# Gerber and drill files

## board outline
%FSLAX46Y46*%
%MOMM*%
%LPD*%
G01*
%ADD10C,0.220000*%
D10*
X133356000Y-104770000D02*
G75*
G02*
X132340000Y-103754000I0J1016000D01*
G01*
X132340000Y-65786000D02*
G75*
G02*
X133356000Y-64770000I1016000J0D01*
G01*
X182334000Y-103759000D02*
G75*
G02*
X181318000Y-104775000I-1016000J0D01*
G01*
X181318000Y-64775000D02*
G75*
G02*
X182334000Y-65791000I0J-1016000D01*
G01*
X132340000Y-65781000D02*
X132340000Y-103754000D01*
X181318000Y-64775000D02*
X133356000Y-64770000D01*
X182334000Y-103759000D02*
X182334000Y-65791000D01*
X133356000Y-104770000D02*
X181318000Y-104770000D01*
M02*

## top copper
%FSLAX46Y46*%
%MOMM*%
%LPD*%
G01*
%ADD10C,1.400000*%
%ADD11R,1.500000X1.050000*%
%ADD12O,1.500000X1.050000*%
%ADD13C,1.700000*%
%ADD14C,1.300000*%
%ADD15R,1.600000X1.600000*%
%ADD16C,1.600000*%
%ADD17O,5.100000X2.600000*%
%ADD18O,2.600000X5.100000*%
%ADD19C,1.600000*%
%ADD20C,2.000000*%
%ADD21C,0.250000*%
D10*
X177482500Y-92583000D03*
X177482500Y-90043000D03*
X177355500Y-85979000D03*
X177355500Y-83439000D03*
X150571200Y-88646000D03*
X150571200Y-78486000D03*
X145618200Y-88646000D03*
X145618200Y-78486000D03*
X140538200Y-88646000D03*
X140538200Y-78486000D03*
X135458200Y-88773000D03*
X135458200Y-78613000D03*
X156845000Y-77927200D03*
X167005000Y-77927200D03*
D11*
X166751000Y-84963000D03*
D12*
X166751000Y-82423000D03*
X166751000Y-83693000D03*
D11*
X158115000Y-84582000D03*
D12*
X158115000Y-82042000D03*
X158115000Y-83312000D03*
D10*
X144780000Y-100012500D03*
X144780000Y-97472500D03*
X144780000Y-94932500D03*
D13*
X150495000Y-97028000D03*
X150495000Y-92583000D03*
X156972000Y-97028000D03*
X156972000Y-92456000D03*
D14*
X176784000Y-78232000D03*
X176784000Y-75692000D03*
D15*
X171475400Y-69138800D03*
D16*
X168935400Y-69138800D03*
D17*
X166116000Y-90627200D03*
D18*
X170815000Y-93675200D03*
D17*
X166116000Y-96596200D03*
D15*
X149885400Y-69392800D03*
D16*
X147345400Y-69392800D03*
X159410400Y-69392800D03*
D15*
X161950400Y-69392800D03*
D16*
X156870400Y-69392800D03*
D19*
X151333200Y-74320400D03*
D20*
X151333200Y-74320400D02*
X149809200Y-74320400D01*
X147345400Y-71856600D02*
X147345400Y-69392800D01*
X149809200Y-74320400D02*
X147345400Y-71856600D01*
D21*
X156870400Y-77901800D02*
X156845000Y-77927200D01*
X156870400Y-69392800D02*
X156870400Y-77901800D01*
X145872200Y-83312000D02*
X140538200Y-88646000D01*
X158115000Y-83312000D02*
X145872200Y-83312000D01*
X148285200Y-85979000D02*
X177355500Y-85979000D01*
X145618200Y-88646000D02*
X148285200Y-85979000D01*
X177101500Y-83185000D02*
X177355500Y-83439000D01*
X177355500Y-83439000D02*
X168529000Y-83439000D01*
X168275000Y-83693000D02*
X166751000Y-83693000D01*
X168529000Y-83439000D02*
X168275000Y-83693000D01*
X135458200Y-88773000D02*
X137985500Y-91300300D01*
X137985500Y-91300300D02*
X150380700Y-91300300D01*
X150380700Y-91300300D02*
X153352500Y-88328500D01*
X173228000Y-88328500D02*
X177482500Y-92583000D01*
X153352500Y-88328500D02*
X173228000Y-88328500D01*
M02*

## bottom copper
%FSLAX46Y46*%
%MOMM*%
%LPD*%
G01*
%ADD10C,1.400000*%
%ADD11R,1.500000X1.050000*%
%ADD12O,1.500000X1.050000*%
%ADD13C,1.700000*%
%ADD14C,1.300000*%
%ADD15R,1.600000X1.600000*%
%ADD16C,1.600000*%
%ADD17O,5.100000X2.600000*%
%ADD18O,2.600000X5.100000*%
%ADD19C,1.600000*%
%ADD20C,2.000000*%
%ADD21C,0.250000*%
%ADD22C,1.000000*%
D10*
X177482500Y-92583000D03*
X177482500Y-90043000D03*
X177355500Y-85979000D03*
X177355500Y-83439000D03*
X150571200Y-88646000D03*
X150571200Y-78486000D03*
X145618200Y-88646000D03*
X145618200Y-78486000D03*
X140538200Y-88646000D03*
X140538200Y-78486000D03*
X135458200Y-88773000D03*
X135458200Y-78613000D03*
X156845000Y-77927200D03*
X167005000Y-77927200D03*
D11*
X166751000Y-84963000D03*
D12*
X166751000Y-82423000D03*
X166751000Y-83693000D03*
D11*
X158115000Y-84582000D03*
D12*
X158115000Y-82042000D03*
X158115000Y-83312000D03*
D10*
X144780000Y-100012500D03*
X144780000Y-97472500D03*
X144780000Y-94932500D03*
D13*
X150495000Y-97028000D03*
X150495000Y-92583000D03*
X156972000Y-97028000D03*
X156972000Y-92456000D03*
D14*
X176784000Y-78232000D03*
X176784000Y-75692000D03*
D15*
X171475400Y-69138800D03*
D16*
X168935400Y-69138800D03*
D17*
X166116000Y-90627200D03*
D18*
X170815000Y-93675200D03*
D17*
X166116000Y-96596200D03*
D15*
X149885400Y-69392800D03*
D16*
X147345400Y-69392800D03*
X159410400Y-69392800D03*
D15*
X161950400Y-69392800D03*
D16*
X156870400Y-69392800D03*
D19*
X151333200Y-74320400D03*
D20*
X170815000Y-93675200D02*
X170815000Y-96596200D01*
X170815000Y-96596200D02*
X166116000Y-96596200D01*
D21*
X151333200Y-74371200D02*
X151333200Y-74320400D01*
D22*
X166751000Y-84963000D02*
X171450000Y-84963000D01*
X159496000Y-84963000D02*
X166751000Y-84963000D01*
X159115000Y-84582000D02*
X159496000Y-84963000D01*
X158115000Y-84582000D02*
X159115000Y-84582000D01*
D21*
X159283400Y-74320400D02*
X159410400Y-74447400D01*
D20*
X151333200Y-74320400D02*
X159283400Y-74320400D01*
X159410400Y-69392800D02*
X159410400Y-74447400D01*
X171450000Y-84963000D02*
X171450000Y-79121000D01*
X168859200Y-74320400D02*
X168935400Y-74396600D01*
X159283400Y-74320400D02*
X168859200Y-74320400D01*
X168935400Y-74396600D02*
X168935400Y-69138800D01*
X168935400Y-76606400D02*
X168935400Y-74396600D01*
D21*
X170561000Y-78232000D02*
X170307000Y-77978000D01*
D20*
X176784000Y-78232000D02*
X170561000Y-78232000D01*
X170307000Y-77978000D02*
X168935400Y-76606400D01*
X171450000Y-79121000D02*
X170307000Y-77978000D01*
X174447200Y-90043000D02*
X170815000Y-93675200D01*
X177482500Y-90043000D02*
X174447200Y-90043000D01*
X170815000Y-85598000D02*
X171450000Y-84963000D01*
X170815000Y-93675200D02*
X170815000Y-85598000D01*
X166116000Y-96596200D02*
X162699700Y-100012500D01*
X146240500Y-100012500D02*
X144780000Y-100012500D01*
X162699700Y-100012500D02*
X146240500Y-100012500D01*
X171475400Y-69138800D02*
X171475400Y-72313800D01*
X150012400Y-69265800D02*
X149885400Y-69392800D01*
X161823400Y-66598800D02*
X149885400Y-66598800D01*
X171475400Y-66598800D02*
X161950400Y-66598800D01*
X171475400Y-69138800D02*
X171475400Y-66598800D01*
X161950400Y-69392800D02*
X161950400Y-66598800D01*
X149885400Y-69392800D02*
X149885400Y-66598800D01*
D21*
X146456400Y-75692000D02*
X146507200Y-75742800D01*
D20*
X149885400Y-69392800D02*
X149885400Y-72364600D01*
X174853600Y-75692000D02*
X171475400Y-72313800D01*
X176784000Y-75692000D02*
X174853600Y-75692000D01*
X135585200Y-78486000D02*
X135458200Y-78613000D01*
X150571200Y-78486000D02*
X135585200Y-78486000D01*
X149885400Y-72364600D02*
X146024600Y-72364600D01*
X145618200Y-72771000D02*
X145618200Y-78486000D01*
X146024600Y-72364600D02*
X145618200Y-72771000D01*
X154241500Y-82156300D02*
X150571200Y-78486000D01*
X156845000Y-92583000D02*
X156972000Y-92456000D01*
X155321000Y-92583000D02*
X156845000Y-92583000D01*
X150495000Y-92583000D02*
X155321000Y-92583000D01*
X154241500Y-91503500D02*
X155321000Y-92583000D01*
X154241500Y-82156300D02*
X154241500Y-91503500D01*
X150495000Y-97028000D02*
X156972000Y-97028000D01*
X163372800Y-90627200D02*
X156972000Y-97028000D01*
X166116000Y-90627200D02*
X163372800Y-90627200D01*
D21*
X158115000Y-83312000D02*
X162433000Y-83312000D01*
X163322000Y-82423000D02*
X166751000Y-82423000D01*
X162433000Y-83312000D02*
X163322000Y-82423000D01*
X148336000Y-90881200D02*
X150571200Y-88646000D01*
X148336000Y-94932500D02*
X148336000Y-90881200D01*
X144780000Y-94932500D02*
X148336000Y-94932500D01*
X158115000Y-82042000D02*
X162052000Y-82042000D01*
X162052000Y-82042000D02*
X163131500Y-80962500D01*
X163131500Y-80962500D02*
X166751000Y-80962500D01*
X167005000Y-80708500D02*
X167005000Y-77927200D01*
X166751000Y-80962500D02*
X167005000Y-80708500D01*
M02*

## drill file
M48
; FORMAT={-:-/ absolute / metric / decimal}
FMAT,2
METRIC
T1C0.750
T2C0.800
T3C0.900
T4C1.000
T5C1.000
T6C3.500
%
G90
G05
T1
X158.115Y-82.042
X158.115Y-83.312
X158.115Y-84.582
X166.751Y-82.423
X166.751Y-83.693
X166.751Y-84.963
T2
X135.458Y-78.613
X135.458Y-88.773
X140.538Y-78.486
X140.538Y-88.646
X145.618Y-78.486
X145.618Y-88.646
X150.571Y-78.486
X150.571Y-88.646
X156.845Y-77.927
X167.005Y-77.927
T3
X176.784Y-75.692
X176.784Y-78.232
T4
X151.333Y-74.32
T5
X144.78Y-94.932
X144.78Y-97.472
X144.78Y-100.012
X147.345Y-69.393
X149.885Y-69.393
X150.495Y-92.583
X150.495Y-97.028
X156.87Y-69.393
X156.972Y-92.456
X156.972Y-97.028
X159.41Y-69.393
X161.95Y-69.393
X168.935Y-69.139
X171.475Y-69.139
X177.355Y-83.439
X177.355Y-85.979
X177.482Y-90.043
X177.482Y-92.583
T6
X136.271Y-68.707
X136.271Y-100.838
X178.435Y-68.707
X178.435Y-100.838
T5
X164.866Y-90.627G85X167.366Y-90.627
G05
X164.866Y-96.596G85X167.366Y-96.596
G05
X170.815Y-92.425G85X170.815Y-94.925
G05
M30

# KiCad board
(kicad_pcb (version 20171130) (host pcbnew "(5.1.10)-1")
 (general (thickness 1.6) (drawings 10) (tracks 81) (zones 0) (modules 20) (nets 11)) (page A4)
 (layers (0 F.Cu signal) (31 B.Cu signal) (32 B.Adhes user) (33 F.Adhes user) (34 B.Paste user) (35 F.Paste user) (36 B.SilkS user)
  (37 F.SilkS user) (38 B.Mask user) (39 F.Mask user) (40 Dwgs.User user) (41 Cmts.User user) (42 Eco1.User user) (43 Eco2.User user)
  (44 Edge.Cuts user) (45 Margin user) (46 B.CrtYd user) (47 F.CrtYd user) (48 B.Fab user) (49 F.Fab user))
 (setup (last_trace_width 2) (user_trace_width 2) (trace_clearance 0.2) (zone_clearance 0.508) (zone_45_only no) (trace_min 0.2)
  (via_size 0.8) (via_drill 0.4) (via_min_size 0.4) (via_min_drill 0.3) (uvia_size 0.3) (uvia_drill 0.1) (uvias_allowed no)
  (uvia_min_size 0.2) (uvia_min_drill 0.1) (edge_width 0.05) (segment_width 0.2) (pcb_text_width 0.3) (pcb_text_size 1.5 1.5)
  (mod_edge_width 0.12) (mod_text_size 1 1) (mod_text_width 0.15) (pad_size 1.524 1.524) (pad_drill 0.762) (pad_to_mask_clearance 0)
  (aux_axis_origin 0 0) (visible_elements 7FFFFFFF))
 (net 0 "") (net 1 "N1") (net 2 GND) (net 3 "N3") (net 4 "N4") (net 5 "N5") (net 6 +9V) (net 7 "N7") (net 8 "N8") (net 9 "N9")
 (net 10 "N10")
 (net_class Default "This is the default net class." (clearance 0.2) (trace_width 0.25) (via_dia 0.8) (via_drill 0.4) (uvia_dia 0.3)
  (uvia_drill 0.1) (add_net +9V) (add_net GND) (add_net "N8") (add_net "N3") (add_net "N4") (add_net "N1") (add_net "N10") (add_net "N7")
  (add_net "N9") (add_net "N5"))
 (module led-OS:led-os (layer F.Cu) (at 177.4825 91.313 90)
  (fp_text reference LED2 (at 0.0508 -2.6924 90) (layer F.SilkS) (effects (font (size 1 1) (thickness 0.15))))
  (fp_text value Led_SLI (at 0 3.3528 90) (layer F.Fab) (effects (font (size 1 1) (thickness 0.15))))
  (pad 1 thru_hole circle (at -1.27 0 180) (size 1.4 1.4) (drill 1) (layers *.Cu *.Mask) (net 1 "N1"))
  (pad 2 thru_hole circle (at 1.27 0 180) (size 1.4 1.4) (drill 1) (layers *.Cu *.Mask) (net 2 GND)))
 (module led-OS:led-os (layer F.Cu) (at 177.3555 84.709 90)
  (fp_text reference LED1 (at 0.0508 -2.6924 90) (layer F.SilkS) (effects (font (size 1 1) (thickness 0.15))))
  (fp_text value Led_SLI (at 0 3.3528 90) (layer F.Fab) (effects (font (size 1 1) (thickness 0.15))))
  (pad 1 thru_hole circle (at -1.27 0 180) (size 1.4 1.4) (drill 1) (layers *.Cu *.Mask) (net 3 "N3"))
  (pad 2 thru_hole circle (at 1.27 0 180) (size 1.4 1.4) (drill 1) (layers *.Cu *.Mask) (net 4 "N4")))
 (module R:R (layer F.Cu) (at 150.622 78.486 270)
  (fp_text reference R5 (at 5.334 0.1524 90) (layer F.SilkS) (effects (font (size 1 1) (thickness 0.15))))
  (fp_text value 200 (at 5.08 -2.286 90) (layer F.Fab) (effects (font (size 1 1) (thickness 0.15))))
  (pad 2 thru_hole circle (at 10.16 0.0508 270) (size 1.4 1.4) (drill 0.8) (layers *.Cu *.Mask) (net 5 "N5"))
  (pad 1 thru_hole circle (at 0 0.0508 270) (size 1.4 1.4) (drill 0.8) (layers *.Cu *.Mask) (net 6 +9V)))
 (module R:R (layer F.Cu) (at 145.669 78.486 270)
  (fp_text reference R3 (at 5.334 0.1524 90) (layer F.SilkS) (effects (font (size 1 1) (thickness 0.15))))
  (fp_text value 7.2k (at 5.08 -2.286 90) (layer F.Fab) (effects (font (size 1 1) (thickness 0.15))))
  (pad 2 thru_hole circle (at 10.16 0.0508 270) (size 1.4 1.4) (drill 0.8) (layers *.Cu *.Mask) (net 3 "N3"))
  (pad 1 thru_hole circle (at 0 0.0508 270) (size 1.4 1.4) (drill 0.8) (layers *.Cu *.Mask) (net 6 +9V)))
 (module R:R (layer F.Cu) (at 140.589 78.486 270)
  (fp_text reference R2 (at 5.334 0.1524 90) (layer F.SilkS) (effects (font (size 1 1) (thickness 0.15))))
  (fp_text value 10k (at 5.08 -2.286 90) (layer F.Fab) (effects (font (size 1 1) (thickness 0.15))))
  (pad 2 thru_hole circle (at 10.16 0.0508 270) (size 1.4 1.4) (drill 0.8) (layers *.Cu *.Mask) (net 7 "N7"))
  (pad 1 thru_hole circle (at 0 0.0508 270) (size 1.4 1.4) (drill 0.8) (layers *.Cu *.Mask) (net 6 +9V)))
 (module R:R (layer F.Cu) (at 135.509 78.613 270)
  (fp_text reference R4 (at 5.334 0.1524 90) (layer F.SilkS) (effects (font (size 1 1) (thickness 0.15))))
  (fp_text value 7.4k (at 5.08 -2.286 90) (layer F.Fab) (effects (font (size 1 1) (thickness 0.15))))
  (pad 2 thru_hole circle (at 10.16 0.0508 270) (size 1.4 1.4) (drill 0.8) (layers *.Cu *.Mask) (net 1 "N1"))
  (pad 1 thru_hole circle (at 0 0.0508 270) (size 1.4 1.4) (drill 0.8) (layers *.Cu *.Mask) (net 6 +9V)))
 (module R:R (layer F.Cu) (at 167.005 77.978 180)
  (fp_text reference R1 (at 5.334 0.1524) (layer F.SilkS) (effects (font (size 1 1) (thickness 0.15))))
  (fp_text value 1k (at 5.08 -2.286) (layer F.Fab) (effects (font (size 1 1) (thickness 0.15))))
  (pad 2 thru_hole circle (at 10.16 0.0508 180) (size 1.4 1.4) (drill 0.8) (layers *.Cu *.Mask) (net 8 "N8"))
  (pad 1 thru_hole circle (at 0 0.0508 180) (size 1.4 1.4) (drill 0.8) (layers *.Cu *.Mask) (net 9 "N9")))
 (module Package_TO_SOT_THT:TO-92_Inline (layer F.Cu) (at 166.751 84.963 90)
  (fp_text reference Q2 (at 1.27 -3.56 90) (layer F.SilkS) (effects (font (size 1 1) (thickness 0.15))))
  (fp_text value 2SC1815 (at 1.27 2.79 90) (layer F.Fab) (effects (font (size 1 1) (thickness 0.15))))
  (pad 1 thru_hole rect (at 0 0 90) (size 1.05 1.5) (drill 0.75) (layers *.Cu *.Mask) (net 2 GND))
  (pad 3 thru_hole oval (at 2.54 0 90) (size 1.05 1.5) (drill 0.75) (layers *.Cu *.Mask) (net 7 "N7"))
  (pad 2 thru_hole oval (at 1.27 0 90) (size 1.05 1.5) (drill 0.75) (layers *.Cu *.Mask) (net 4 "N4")))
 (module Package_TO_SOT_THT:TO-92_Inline (layer F.Cu) (at 158.115 84.582 90)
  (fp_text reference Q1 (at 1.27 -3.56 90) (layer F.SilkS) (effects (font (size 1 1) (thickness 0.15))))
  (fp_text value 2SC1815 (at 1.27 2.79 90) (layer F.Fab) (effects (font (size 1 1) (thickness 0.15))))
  (pad 1 thru_hole rect (at 0 0 90) (size 1.05 1.5) (drill 0.75) (layers *.Cu *.Mask) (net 2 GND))
  (pad 3 thru_hole oval (at 2.54 0 90) (size 1.05 1.5) (drill 0.75) (layers *.Cu *.Mask) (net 9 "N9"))
  (pad 2 thru_hole oval (at 1.27 0 90) (size 1.05 1.5) (drill 0.75) (layers *.Cu *.Mask) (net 7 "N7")))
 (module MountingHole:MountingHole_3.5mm (layer F.Cu) (at 136.271 100.838)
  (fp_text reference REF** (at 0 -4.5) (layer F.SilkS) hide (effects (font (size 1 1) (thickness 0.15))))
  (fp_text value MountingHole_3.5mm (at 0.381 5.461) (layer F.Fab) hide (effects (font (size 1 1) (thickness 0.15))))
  (pad 1 np_thru_hole circle (at 0 0) (size 3.5 3.5) (drill 3.5) (layers *.Cu *.Mask)))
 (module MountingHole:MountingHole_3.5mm (layer F.Cu) (at 136.271 68.707)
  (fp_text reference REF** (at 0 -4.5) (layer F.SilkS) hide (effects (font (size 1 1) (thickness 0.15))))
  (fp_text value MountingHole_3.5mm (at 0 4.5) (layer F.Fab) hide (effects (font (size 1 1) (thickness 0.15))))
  (pad 1 np_thru_hole circle (at 0 0) (size 3.5 3.5) (drill 3.5) (layers *.Cu *.Mask)))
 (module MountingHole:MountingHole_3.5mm (layer F.Cu) (at 178.435 68.707)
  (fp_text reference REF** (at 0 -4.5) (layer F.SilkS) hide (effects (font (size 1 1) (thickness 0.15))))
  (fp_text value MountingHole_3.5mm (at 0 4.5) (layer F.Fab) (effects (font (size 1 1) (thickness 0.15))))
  (pad 1 np_thru_hole circle (at 0 0) (size 3.5 3.5) (drill 3.5) (layers *.Cu *.Mask)))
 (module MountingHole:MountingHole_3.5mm (layer F.Cu) (at 178.435 100.838)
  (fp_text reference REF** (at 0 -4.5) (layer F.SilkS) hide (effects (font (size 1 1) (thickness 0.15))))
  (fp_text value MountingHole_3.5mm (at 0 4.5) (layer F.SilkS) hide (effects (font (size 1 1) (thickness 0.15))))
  (pad 1 np_thru_hole circle (at 0 0) (size 3.5 3.5) (drill 3.5) (layers *.Cu *.Mask)))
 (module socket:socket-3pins (layer F.Cu) (at 144.78 97.4725)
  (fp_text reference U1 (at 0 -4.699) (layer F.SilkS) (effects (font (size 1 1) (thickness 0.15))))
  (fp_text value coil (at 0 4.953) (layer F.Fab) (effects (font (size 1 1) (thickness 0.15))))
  (pad 3 thru_hole circle (at 0 2.54) (size 1.4 1.4) (drill 1) (layers *.Cu *.Mask) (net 2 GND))
  (pad 2 thru_hole circle (at 0 0) (size 1.4 1.4) (drill 1) (layers *.Cu *.Mask))
  (pad 1 thru_hole circle (at 0 -2.54) (size 1.4 1.4) (drill 1) (layers *.Cu *.Mask) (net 5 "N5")))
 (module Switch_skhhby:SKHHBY (layer F.Cu) (at 153.797 94.742 90)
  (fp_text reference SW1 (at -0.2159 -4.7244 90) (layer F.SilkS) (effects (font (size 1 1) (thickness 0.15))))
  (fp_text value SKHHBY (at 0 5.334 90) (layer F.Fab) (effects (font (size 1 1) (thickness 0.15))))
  (pad 1 thru_hole circle (at -2.286 -3.302 90) (size 1.7 1.7) (drill 1) (layers *.Cu *.Mask) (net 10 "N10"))
  (pad 3 thru_hole circle (at 2.159 -3.302 90) (size 1.7 1.7) (drill 1) (layers *.Cu *.Mask) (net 6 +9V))
  (pad 2 thru_hole circle (at -2.286 3.175 90) (size 1.7 1.7) (drill 1) (layers *.Cu *.Mask) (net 10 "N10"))
  (pad 4 thru_hole circle (at 2.286 3.175 90) (size 1.7 1.7) (drill 1) (layers *.Cu *.Mask) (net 6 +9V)))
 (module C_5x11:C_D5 (layer F.Cu) (at 176.784 76.962 270)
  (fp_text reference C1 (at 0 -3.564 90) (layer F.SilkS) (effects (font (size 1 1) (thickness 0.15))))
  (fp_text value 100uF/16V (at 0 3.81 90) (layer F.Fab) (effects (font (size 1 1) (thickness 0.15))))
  (pad 2 thru_hole circle (at 1.27 0 270) (size 1.3 1.3) (drill 0.9) (layers *.Cu *.Mask) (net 2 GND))
  (pad 1 thru_hole circle (at -1.27 0 270) (size 1.3 1.3) (drill 0.9) (layers *.Cu *.Mask) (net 6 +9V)))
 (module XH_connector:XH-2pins (layer F.Cu) (at 170.0784 69.1388 270)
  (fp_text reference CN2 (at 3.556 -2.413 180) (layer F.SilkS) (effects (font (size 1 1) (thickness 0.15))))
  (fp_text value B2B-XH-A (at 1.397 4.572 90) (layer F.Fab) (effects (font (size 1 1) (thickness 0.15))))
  (pad 1 thru_hole rect (at 0 -1.397 270) (size 1.6 1.6) (drill 1) (layers *.Cu *.Mask) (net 6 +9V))
  (pad 2 thru_hole circle (at 0 1.143 270) (size 1.6 1.6) (drill 1) (layers *.Cu *.Mask) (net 2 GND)))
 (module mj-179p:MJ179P (layer F.Cu) (at 166.116 90.6272)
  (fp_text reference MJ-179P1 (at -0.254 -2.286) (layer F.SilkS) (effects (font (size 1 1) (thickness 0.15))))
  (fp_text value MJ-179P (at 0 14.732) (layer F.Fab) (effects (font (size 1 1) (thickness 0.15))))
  (pad 1 thru_hole oval (at 0 0 90) (size 2.6 5.1) (drill oval 1 3.5) (layers *.Cu *.Mask) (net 10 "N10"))
  (pad 3 thru_hole oval (at 4.699 3.048) (size 2.6 5.1) (drill oval 1 3.5) (layers *.Cu *.Mask) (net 2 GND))
  (pad 2 thru_hole oval (at 0 5.969 90) (size 2.6 5.1) (drill oval 1 3.5) (layers *.Cu *.Mask) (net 2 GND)))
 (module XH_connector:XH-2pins (layer F.Cu) (at 148.4884 69.3928 270)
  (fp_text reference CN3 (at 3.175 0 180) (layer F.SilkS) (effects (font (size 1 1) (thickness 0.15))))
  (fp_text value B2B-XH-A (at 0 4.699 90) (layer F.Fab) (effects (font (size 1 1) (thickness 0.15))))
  (pad 1 thru_hole rect (at 0 -1.397 270) (size 1.6 1.6) (drill 1) (layers *.Cu *.Mask) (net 6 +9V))
  (pad 2 thru_hole circle (at 0 1.143 270) (size 1.6 1.6) (drill 1) (layers *.Cu *.Mask) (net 2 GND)))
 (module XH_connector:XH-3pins (layer F.Cu) (at 159.4104 69.3928 270)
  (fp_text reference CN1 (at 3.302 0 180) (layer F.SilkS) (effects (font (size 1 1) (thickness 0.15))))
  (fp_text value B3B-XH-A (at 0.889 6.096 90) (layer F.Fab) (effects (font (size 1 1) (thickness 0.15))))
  (pad 2 thru_hole circle (at 0 0 270) (size 1.6 1.6) (drill 1) (layers *.Cu *.Mask) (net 2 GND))
  (pad 1 thru_hole rect (at 0 -2.54 270) (size 1.6 1.6) (drill 1) (layers *.Cu *.Mask) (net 6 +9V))
  (pad 3 thru_hole circle (at 0 2.54 270) (size 1.6 1.6) (drill 1) (layers *.Cu *.Mask) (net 8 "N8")))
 (gr_arc (start 133.356 103.754) (end 132.34 103.754) (angle -90) (layer Edge.Cuts) (width 0.22))
 (gr_arc (start 133.356 65.786) (end 133.356 64.77) (angle -90) (layer Edge.Cuts) (width 0.22))
 (gr_arc (start 181.318 103.759) (end 181.318 104.775) (angle -90) (layer Edge.Cuts) (width 0.22))
 (gr_arc (start 181.318 65.791) (end 182.334 65.791) (angle -90) (layer Edge.Cuts) (width 0.22))
 (gr_line (start 132.34 65.781) (end 132.34 103.754) (layer Edge.Cuts) (width 0.22))
 (gr_line (start 181.318 64.775) (end 133.356 64.77) (layer Edge.Cuts) (width 0.22))
 (gr_line (start 182.334 103.759) (end 182.334 65.791) (layer Edge.Cuts) (width 0.22))
 (gr_line (start 133.356 104.77) (end 181.318 104.77) (layer Edge.Cuts) (width 0.22))
 (segment (start 170.815 93.6752) (end 170.815 96.5962) (width 2) (layer B.Cu) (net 2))
 (segment (start 170.815 96.5962) (end 166.116 96.5962) (width 2) (layer B.Cu) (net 2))
 (via (at 151.3332 74.3204) (size 1.6) (drill 1) (layers F.Cu B.Cu) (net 2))
 (segment (start 151.3332 74.3712) (end 151.3332 74.3204) (width 0.25) (layer B.Cu) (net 2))
 (segment (start 151.3332 74.3204) (end 149.8092 74.3204) (width 2) (layer F.Cu) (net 2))
 (segment (start 147.3454 71.8566) (end 147.3454 69.3928) (width 2) (layer F.Cu) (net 2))
 (segment (start 149.8092 74.3204) (end 147.3454 71.8566) (width 2) (layer F.Cu) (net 2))
 (segment (start 166.751 84.963) (end 171.45 84.963) (width 1) (layer B.Cu) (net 2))
 (segment (start 159.496 84.963) (end 166.751 84.963) (width 1) (layer B.Cu) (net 2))
 (segment (start 159.115 84.582) (end 159.496 84.963) (width 1) (layer B.Cu) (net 2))
 (segment (start 158.115 84.582) (end 159.115 84.582) (width 1) (layer B.Cu) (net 2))
 (segment (start 159.2834 74.3204) (end 159.4104 74.4474) (width 0.25) (layer B.Cu) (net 2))
 (segment (start 151.3332 74.3204) (end 159.2834 74.3204) (width 2) (layer B.Cu) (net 2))
 (segment (start 159.4104 69.3928) (end 159.4104 74.4474) (width 2) (layer B.Cu) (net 2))
 (segment (start 171.45 84.963) (end 171.45 79.121) (width 2) (layer B.Cu) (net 2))
 (segment (start 168.8592 74.3204) (end 168.9354 74.3966) (width 2) (layer B.Cu) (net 2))
 (segment (start 159.2834 74.3204) (end 168.8592 74.3204) (width 2) (layer B.Cu) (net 2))
 (segment (start 168.9354 74.3966) (end 168.9354 69.1388) (width 2) (layer B.Cu) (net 2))
 (segment (start 168.9354 76.6064) (end 168.9354 74.3966) (width 2) (layer B.Cu) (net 2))
 (segment (start 170.561 78.232) (end 170.307 77.978) (width 0.25) (layer B.Cu) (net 2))
 (segment (start 176.784 78.232) (end 170.561 78.232) (width 2) (layer B.Cu) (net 2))
 (segment (start 170.307 77.978) (end 168.9354 76.6064) (width 2) (layer B.Cu) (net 2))
 (segment (start 171.45 79.121) (end 170.307 77.978) (width 2) (layer B.Cu) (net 2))
 (segment (start 174.4472 90.043) (end 170.815 93.6752) (width 2) (layer B.Cu) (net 2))
 (segment (start 177.4825 90.043) (end 174.4472 90.043) (width 2) (layer B.Cu) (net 2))
 (segment (start 170.815 85.598) (end 171.45 84.963) (width 2) (layer B.Cu) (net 2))
 (segment (start 170.815 93.6752) (end 170.815 85.598) (width 2) (layer B.Cu) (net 2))
 (segment (start 166.116 96.5962) (end 162.6997 100.0125) (width 2) (layer B.Cu) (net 2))
 (segment (start 146.2405 100.0125) (end 144.78 100.0125) (width 2) (layer B.Cu) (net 2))
 (segment (start 162.6997 100.0125) (end 146.2405 100.0125) (width 2) (layer B.Cu) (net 2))
 (segment (start 171.4754 69.1388) (end 171.4754 72.3138) (width 2) (layer B.Cu) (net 6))
 (segment (start 150.0124 69.2658) (end 149.8854 69.3928) (width 2) (layer B.Cu) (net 6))
 (segment (start 161.8234 66.5988) (end 149.8854 66.5988) (width 2) (layer B.Cu) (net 6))
 (segment (start 171.4754 66.5988) (end 161.9504 66.5988) (width 2) (layer B.Cu) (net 6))
 (segment (start 171.4754 69.1388) (end 171.4754 66.5988) (width 2) (layer B.Cu) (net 6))
 (segment (start 161.9504 69.3928) (end 161.9504 66.5988) (width 2) (layer B.Cu) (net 6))
 (segment (start 149.8854 69.3928) (end 149.8854 66.5988) (width 2) (layer B.Cu) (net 6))
 (segment (start 146.4564 75.692) (end 146.5072 75.7428) (width 0.25) (layer B.Cu) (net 6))
 (segment (start 149.8854 69.3928) (end 149.8854 72.3646) (width 2) (layer B.Cu) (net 6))
 (segment (start 174.8536 75.692) (end 171.4754 72.3138) (width 2) (layer B.Cu) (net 6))
 (segment (start 176.784 75.692) (end 174.8536 75.692) (width 2) (layer B.Cu) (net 6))
 (segment (start 135.5852 78.486) (end 135.4582 78.613) (width 2) (layer B.Cu) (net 6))
 (segment (start 150.5712 78.486) (end 135.5852 78.486) (width 2) (layer B.Cu) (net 6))
 (segment (start 149.8854 72.3646) (end 146.0246 72.3646) (width 2) (layer B.Cu) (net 6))
 (segment (start 145.6182 72.771) (end 145.6182 78.486) (width 2) (layer B.Cu) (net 6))
 (segment (start 146.0246 72.3646) (end 145.6182 72.771) (width 2) (layer B.Cu) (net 6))
 (segment (start 154.2415 82.1563) (end 150.5712 78.486) (width 2) (layer B.Cu) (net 6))
 (segment (start 156.845 92.583) (end 156.972 92.456) (width 2) (layer B.Cu) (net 6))
 (segment (start 155.321 92.583) (end 156.845 92.583) (width 2) (layer B.Cu) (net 6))
 (segment (start 150.495 92.583) (end 155.321 92.583) (width 2) (layer B.Cu) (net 6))
 (segment (start 154.2415 91.5035) (end 155.321 92.583) (width 2) (layer B.Cu) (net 6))
 (segment (start 154.2415 82.1563) (end 154.2415 91.5035) (width 2) (layer B.Cu) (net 6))
 (segment (start 156.8704 77.9018) (end 156.845 77.9272) (width 0.25) (layer F.Cu) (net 8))
 (segment (start 156.8704 69.3928) (end 156.8704 77.9018) (width 0.25) (layer F.Cu) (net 8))
 (segment (start 150.495 97.028) (end 156.972 97.028) (width 2) (layer B.Cu) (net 10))
 (segment (start 163.3728 90.6272) (end 156.972 97.028) (width 2) (layer B.Cu) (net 10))
 (segment (start 166.116 90.6272) (end 163.3728 90.6272) (width 2) (layer B.Cu) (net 10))
 (segment (start 158.115 83.312) (end 162.433 83.312) (width 0.25) (layer B.Cu) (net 7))
 (segment (start 163.322 82.423) (end 166.751 82.423) (width 0.25) (layer B.Cu) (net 7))
 (segment (start 162.433 83.312) (end 163.322 82.423) (width 0.25) (layer B.Cu) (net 7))
 (segment (start 145.8722 83.312) (end 140.5382 88.646) (width 0.25) (layer F.Cu) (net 7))
 (segment (start 158.115 83.312) (end 145.8722 83.312) (width 0.25) (layer F.Cu) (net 7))
 (segment (start 148.336 90.8812) (end 150.5712 88.646) (width 0.25) (layer B.Cu) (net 5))
 (segment (start 148.336 94.9325) (end 148.336 90.8812) (width 0.25) (layer B.Cu) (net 5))
 (segment (start 144.78 94.9325) (end 148.336 94.9325) (width 0.25) (layer B.Cu) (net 5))
 (segment (start 148.2852 85.979) (end 177.3555 85.979) (width 0.25) (layer F.Cu) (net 3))
 (segment (start 145.6182 88.646) (end 148.2852 85.979) (width 0.25) (layer F.Cu) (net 3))
 (segment (start 177.1015 83.185) (end 177.3555 83.439) (width 0.25) (layer F.Cu) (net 4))
 (segment (start 177.3555 83.439) (end 168.529 83.439) (width 0.25) (layer F.Cu) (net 4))
 (segment (start 168.275 83.693) (end 166.751 83.693) (width 0.25) (layer F.Cu) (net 4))
 (segment (start 168.529 83.439) (end 168.275 83.693) (width 0.25) (layer F.Cu) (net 4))
 (segment (start 158.115 82.042) (end 162.052 82.042) (width 0.25) (layer B.Cu) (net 9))
 (segment (start 162.052 82.042) (end 163.1315 80.9625) (width 0.25) (layer B.Cu) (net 9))
 (segment (start 163.1315 80.9625) (end 166.751 80.9625) (width 0.25) (layer B.Cu) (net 9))
 (segment (start 167.005 80.7085) (end 167.005 77.9272) (width 0.25) (layer B.Cu) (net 9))
 (segment (start 166.751 80.9625) (end 167.005 80.7085) (width 0.25) (layer B.Cu) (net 9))
 (segment (start 135.4582 88.773) (end 137.9855 91.3003) (width 0.25) (layer F.Cu) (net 1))
 (segment (start 137.9855 91.3003) (end 150.3807 91.3003) (width 0.25) (layer F.Cu) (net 1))
 (segment (start 150.3807 91.3003) (end 153.3525 88.3285) (width 0.25) (layer F.Cu) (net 1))
 (segment (start 173.228 88.3285) (end 177.4825 92.583) (width 0.25) (layer F.Cu) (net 1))
 (segment (start 153.3525 88.3285) (end 173.228 88.3285) (width 0.25) (layer F.Cu) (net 1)))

